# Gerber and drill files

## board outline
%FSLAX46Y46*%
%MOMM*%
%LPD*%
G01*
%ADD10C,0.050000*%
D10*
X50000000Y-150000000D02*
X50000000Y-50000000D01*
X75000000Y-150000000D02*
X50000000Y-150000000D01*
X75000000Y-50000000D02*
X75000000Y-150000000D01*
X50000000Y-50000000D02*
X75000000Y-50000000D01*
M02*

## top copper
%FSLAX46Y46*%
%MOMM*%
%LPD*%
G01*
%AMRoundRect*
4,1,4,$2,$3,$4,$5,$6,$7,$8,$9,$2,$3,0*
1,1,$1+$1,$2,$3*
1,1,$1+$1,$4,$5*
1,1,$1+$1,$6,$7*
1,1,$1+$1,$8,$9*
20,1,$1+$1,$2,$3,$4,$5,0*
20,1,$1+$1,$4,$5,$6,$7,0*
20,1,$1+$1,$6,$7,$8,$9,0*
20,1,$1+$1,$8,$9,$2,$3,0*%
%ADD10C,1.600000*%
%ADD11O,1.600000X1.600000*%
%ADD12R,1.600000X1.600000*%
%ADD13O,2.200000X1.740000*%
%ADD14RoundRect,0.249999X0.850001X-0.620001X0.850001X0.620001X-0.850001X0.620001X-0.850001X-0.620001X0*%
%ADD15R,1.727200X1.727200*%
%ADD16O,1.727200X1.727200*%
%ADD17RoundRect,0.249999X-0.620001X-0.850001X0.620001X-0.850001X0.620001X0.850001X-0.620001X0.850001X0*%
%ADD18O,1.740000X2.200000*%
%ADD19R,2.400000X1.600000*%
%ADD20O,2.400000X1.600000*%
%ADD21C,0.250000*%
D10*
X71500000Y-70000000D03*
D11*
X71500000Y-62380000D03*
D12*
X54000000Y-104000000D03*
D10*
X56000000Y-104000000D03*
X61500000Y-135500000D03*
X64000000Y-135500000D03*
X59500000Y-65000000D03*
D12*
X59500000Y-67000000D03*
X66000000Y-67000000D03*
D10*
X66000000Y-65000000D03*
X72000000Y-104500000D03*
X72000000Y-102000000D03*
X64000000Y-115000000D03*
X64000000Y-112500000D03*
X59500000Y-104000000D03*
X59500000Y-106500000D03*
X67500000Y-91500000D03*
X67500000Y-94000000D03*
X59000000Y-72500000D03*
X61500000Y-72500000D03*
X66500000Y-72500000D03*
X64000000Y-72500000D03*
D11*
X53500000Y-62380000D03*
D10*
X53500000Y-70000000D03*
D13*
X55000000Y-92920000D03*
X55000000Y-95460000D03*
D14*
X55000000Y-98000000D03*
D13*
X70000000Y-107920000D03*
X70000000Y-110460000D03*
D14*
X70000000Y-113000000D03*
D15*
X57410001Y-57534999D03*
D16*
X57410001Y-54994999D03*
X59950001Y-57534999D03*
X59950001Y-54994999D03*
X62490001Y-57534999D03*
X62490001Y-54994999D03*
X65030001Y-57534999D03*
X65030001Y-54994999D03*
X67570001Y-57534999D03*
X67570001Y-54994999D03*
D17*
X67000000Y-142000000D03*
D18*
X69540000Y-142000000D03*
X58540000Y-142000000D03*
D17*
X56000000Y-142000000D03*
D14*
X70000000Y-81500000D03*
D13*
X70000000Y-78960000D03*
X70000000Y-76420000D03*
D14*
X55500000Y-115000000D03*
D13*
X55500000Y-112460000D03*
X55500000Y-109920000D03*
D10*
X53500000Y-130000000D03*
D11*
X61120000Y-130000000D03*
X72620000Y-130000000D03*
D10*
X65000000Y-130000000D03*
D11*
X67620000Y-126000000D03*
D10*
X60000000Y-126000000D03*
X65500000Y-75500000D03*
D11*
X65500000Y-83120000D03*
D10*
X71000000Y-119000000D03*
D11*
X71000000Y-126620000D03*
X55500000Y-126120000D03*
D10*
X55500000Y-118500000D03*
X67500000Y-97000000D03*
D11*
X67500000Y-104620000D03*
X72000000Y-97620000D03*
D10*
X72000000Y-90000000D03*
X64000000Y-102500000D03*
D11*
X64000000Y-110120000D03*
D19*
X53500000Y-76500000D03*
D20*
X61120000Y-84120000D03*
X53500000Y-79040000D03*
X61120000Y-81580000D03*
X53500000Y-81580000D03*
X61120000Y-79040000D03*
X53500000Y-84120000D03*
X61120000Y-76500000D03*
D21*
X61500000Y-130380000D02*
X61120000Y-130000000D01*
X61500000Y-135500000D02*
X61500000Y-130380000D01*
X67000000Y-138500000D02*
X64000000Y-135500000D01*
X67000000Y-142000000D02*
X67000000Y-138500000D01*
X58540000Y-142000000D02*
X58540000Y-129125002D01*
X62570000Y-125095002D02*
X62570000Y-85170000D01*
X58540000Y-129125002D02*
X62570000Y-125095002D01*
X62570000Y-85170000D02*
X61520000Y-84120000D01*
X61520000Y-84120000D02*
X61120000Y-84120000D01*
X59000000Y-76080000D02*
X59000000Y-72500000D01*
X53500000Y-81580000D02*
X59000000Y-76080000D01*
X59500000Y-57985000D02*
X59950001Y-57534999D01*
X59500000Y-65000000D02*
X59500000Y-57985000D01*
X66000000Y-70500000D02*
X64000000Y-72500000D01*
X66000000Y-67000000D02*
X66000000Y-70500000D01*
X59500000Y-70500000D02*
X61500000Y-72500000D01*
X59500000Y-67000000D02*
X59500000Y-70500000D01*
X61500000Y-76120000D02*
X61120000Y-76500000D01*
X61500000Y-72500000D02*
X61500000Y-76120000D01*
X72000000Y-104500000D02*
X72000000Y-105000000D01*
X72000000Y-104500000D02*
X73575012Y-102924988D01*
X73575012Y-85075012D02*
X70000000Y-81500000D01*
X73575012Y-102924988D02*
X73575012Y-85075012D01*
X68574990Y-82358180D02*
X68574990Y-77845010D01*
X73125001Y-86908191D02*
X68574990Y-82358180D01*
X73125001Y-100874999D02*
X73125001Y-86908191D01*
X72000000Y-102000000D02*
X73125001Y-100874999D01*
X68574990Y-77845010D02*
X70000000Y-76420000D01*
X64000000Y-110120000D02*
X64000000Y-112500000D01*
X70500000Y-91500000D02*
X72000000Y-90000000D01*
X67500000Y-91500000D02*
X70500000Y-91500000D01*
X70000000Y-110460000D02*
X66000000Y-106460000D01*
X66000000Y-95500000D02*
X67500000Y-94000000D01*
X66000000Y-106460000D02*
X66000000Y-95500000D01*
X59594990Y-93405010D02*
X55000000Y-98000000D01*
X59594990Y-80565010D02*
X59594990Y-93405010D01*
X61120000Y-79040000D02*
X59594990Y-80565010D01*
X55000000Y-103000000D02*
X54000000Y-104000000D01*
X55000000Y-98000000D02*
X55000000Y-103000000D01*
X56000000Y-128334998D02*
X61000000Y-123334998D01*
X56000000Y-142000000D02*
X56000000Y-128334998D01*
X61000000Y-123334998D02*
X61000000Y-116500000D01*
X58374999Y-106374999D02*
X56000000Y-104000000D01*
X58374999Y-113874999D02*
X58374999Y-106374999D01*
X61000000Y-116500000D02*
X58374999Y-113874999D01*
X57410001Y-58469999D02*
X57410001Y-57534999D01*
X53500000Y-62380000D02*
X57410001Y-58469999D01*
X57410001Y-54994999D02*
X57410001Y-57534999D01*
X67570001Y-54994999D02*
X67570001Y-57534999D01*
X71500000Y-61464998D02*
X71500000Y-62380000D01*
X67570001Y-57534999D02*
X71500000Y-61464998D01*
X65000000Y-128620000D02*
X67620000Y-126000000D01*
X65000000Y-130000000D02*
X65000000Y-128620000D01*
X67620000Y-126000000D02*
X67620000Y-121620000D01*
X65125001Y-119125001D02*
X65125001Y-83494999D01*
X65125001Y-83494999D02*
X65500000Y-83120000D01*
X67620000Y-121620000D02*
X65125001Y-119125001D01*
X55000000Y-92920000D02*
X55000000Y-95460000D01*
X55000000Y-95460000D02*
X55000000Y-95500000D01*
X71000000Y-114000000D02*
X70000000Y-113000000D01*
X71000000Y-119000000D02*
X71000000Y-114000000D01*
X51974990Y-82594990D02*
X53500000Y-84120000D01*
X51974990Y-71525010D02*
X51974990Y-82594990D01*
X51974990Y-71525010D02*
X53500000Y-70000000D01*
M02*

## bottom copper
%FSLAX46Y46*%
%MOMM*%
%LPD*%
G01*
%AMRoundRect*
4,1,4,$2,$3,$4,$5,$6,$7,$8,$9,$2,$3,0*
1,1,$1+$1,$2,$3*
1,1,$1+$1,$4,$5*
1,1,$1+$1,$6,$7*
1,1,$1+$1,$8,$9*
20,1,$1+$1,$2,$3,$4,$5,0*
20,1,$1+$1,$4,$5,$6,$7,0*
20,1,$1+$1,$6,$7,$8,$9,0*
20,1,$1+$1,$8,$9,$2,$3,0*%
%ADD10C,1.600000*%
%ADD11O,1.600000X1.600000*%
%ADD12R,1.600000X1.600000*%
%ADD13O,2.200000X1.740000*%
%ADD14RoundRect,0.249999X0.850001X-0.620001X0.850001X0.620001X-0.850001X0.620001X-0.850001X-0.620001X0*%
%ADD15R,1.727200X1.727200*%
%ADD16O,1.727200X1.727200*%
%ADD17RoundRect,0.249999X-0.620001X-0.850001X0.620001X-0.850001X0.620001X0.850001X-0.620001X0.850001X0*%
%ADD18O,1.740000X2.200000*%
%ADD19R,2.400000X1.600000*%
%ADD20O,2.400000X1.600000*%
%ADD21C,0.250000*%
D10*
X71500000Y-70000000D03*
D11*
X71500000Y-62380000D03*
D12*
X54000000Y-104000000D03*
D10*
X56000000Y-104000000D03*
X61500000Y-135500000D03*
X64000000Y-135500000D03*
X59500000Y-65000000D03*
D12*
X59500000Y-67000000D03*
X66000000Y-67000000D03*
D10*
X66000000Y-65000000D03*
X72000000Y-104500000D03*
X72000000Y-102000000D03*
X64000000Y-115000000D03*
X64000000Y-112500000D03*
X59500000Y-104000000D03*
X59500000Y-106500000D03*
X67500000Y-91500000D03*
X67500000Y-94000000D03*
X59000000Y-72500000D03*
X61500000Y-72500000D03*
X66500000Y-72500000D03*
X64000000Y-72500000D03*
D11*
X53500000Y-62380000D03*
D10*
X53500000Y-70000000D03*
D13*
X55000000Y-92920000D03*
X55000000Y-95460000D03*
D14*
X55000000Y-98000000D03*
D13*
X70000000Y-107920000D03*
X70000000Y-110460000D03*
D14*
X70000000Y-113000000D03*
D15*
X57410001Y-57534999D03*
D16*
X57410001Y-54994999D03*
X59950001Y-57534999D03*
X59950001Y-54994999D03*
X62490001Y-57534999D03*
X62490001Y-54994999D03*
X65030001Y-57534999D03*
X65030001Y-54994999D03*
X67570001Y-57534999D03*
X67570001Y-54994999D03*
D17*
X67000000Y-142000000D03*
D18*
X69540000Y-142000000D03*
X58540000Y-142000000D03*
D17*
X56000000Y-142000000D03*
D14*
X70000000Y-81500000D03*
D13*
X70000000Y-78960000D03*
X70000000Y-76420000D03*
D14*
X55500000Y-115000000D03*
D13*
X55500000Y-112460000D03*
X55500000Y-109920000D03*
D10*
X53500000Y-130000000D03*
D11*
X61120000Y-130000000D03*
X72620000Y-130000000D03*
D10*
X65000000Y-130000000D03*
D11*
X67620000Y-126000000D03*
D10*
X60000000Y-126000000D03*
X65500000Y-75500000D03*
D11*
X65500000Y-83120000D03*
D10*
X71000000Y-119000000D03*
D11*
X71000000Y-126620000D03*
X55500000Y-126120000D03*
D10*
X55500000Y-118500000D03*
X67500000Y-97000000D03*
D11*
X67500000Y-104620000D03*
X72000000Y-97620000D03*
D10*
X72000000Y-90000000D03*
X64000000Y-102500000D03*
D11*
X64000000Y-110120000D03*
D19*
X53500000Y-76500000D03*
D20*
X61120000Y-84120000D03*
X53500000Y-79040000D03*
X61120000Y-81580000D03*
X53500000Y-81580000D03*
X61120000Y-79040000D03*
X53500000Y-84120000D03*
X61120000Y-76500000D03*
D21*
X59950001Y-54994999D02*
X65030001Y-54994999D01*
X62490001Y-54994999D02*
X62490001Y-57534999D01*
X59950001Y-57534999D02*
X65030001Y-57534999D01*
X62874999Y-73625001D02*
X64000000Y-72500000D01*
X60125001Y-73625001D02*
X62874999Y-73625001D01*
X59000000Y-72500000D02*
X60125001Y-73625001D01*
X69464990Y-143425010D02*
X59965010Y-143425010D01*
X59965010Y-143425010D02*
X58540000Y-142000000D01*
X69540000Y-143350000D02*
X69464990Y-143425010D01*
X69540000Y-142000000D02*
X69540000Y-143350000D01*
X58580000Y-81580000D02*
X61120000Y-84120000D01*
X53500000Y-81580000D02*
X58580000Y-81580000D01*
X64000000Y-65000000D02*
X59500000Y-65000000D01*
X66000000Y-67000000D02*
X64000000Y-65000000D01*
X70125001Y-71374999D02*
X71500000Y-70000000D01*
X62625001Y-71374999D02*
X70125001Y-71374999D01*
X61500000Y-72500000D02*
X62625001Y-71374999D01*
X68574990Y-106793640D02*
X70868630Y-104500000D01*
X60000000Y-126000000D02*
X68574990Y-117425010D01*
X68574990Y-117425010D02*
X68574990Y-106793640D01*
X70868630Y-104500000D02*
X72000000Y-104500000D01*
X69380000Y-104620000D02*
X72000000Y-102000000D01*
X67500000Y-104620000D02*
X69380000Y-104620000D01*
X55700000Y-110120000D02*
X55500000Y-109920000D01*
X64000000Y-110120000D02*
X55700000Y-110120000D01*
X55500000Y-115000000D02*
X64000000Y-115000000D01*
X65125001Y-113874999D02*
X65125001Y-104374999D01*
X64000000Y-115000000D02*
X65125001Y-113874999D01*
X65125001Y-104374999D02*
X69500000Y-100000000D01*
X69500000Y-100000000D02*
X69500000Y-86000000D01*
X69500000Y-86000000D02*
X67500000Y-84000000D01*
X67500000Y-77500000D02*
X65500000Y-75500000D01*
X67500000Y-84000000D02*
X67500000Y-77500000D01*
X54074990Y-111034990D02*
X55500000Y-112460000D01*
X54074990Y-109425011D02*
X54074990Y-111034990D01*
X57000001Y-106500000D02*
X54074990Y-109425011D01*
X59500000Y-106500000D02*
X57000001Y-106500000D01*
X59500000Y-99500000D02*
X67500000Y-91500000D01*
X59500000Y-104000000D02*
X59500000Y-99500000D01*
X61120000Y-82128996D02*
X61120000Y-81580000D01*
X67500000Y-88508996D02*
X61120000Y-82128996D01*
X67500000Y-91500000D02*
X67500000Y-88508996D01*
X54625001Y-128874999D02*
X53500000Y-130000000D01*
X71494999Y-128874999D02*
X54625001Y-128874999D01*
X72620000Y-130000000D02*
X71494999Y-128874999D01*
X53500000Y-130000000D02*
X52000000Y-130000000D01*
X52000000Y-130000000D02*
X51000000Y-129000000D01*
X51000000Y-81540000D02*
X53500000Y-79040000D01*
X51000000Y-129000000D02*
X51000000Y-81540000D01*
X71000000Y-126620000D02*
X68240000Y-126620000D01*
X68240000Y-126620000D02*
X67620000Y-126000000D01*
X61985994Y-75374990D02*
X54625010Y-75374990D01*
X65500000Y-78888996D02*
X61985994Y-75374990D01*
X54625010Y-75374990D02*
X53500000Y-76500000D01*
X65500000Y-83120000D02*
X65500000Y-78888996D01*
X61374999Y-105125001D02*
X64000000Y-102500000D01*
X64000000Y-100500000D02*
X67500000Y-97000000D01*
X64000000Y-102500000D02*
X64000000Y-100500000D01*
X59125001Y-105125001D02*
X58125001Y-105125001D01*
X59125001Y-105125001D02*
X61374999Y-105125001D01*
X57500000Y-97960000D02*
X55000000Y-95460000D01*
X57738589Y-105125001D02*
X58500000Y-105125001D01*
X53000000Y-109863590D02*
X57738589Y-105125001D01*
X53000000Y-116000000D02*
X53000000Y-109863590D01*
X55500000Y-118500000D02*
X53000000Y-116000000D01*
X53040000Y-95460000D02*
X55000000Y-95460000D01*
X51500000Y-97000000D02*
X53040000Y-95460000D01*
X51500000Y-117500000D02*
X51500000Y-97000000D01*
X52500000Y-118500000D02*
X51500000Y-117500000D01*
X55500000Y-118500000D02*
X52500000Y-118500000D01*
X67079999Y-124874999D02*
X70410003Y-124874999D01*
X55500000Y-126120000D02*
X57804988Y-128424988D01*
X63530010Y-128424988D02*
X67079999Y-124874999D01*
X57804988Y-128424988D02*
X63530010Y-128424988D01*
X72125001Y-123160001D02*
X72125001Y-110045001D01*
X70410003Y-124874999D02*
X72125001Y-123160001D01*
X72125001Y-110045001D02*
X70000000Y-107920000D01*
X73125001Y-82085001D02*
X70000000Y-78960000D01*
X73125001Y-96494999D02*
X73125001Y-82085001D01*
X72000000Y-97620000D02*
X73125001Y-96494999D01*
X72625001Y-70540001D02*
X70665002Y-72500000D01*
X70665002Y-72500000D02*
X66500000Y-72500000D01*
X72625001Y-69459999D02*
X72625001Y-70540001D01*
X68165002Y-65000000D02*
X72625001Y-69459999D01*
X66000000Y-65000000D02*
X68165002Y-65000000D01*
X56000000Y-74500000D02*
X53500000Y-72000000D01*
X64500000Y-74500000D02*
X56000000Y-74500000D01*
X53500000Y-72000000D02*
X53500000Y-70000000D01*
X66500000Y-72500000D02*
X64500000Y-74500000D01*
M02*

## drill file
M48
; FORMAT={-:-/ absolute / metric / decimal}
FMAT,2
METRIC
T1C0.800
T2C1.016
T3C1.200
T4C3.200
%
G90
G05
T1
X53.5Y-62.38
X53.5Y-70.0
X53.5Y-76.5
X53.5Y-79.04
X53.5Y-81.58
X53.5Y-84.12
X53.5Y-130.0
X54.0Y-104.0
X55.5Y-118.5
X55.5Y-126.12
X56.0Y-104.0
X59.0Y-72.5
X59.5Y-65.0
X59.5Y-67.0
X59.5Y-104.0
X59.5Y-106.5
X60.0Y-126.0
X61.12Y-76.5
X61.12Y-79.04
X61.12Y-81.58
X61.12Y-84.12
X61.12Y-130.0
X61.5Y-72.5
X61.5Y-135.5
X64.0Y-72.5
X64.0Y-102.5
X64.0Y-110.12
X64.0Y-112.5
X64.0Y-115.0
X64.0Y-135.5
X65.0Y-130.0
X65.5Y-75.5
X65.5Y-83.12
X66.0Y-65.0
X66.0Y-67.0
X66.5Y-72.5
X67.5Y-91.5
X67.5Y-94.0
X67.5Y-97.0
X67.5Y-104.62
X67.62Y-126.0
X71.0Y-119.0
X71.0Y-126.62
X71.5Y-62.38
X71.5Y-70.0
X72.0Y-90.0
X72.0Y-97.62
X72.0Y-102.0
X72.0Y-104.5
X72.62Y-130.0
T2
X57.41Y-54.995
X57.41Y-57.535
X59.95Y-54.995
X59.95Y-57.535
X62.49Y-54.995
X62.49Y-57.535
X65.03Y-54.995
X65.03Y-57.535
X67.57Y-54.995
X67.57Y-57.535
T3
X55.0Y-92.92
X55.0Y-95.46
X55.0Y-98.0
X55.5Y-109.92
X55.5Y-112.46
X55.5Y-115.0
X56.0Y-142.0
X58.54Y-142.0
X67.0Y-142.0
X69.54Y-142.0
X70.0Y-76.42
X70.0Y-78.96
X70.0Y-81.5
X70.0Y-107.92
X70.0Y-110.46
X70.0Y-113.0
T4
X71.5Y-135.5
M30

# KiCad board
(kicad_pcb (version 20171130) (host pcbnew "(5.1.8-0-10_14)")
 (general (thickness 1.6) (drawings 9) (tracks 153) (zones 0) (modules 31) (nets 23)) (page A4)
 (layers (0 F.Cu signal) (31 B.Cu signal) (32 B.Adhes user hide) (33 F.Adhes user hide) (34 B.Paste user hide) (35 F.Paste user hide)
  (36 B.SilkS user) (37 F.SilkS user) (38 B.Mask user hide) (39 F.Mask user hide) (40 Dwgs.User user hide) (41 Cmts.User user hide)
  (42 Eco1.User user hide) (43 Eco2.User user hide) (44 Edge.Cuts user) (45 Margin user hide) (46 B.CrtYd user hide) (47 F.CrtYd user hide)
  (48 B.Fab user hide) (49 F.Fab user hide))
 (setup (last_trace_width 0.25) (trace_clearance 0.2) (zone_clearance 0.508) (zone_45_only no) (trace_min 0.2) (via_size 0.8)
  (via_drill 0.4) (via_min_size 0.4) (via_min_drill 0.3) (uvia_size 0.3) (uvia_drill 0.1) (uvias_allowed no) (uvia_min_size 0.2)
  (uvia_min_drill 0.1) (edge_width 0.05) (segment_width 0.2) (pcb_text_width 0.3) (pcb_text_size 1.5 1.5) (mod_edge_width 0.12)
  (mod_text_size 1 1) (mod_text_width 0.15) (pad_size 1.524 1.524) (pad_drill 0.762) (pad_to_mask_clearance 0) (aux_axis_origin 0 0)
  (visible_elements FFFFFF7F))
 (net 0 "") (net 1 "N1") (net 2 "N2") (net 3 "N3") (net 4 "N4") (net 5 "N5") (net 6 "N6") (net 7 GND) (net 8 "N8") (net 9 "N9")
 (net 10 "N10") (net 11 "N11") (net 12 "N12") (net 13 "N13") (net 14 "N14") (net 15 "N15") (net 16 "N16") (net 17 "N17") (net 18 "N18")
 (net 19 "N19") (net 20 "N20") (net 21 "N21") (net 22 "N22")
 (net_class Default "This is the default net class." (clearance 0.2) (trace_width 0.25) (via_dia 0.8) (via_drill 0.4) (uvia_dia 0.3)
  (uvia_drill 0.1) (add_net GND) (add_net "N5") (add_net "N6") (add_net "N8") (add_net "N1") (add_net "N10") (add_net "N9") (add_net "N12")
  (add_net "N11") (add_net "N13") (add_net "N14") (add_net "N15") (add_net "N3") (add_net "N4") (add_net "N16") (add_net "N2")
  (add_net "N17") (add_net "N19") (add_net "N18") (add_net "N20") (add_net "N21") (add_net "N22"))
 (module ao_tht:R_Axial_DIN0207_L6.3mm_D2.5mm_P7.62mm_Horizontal (layer F.Cu) (at 71.5 70 90)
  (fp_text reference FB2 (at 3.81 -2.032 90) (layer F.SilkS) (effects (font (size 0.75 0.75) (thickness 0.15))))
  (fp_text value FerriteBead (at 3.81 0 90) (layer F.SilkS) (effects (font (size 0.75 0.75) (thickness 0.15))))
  (pad 1 thru_hole circle (at 0 0 90) (size 1.6 1.6) (drill 0.8) (layers *.Cu *.Mask) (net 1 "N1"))
  (pad 2 thru_hole oval (at 7.62 0 90) (size 1.6 1.6) (drill 0.8) (layers *.Cu *.Mask) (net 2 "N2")))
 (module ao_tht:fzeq (layer B.Cu) (at 62 63 180)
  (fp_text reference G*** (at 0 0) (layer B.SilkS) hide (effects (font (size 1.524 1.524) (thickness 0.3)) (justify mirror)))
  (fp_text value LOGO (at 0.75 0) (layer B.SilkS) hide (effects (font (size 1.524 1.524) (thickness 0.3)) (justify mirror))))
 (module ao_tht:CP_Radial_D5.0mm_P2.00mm (layer F.Cu) (at 54 104)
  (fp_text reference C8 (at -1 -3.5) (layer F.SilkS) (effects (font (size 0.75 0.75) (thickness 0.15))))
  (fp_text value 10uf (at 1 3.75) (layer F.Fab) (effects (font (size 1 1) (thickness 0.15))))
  (pad 1 thru_hole rect (at 0 0) (size 1.6 1.6) (drill 0.8) (layers *.Cu *.Mask) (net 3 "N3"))
  (pad 2 thru_hole circle (at 2 0) (size 1.6 1.6) (drill 0.8) (layers *.Cu *.Mask) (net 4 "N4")))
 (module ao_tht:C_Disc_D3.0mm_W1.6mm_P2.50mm (layer F.Cu) (at 61.5 135.5)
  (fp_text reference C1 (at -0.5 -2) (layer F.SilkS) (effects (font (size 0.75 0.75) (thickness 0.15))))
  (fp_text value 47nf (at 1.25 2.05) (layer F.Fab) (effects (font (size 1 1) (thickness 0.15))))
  (pad 1 thru_hole circle (at 0 0) (size 1.6 1.6) (drill 0.8) (layers *.Cu *.Mask) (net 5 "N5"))
  (pad 2 thru_hole circle (at 2.5 0) (size 1.6 1.6) (drill 0.8) (layers *.Cu *.Mask) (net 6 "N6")))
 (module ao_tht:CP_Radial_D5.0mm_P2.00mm (layer F.Cu) (at 59.5 67 90)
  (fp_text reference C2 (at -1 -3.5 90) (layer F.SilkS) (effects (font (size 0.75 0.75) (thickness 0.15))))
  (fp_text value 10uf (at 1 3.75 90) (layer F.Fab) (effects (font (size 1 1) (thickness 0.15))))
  (pad 2 thru_hole circle (at 2 0 90) (size 1.6 1.6) (drill 0.8) (layers *.Cu *.Mask) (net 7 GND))
  (pad 1 thru_hole rect (at 0 0 90) (size 1.6 1.6) (drill 0.8) (layers *.Cu *.Mask) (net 1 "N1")))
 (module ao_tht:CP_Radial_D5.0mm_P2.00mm (layer F.Cu) (at 66 67 90)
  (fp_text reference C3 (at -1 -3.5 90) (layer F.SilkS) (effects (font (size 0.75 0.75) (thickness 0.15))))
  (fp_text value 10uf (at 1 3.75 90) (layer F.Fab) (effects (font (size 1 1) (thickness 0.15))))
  (pad 1 thru_hole rect (at 0 0 90) (size 1.6 1.6) (drill 0.8) (layers *.Cu *.Mask) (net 7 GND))
  (pad 2 thru_hole circle (at 2 0 90) (size 1.6 1.6) (drill 0.8) (layers *.Cu *.Mask) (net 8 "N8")))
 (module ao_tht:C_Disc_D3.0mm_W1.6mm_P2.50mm (layer F.Cu) (at 72 102 270)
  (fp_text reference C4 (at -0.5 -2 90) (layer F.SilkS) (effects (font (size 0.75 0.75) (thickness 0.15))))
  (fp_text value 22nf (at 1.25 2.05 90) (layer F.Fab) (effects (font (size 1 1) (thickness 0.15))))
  (pad 2 thru_hole circle (at 2.5 0 270) (size 1.6 1.6) (drill 0.8) (layers *.Cu *.Mask) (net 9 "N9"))
  (pad 1 thru_hole circle (at 0 0 270) (size 1.6 1.6) (drill 0.8) (layers *.Cu *.Mask) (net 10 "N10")))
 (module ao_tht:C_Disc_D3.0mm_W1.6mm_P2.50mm (layer F.Cu) (at 64 112.5 270)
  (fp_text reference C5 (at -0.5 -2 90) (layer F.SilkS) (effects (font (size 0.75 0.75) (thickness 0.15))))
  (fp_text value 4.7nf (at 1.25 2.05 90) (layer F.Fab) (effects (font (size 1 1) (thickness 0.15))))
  (pad 2 thru_hole circle (at 2.5 0 270) (size 1.6 1.6) (drill 0.8) (layers *.Cu *.Mask) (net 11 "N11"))
  (pad 1 thru_hole circle (at 0 0 270) (size 1.6 1.6) (drill 0.8) (layers *.Cu *.Mask) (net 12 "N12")))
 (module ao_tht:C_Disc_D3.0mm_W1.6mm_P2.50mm (layer F.Cu) (at 59.5 104 270)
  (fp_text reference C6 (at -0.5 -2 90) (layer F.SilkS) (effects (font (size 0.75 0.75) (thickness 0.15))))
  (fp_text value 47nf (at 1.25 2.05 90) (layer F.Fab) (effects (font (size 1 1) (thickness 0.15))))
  (pad 1 thru_hole circle (at 0 0 270) (size 1.6 1.6) (drill 0.8) (layers *.Cu *.Mask) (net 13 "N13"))
  (pad 2 thru_hole circle (at 2.5 0 270) (size 1.6 1.6) (drill 0.8) (layers *.Cu *.Mask) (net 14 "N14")))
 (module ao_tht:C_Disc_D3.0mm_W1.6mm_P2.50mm (layer F.Cu) (at 67.5 91.5 270)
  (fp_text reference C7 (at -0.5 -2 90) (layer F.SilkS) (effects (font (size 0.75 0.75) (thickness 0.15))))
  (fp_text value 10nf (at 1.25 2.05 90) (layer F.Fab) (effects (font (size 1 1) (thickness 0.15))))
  (pad 1 thru_hole circle (at 0 0 270) (size 1.6 1.6) (drill 0.8) (layers *.Cu *.Mask) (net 13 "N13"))
  (pad 2 thru_hole circle (at 2.5 0 270) (size 1.6 1.6) (drill 0.8) (layers *.Cu *.Mask) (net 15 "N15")))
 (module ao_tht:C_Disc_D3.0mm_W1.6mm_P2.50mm (layer F.Cu) (at 59 72.5)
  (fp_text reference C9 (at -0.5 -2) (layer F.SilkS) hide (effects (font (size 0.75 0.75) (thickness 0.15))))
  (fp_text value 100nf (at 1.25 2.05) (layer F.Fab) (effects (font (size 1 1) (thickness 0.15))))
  (pad 1 thru_hole circle (at 0 0) (size 1.6 1.6) (drill 0.8) (layers *.Cu *.Mask) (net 7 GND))
  (pad 2 thru_hole circle (at 2.5 0) (size 1.6 1.6) (drill 0.8) (layers *.Cu *.Mask) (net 1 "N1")))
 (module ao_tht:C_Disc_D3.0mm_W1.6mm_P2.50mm (layer F.Cu) (at 64 72.5)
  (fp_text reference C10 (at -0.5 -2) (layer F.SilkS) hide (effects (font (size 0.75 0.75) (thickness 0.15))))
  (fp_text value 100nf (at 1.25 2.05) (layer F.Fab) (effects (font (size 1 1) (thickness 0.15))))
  (pad 2 thru_hole circle (at 2.5 0) (size 1.6 1.6) (drill 0.8) (layers *.Cu *.Mask) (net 8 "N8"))
  (pad 1 thru_hole circle (at 0 0) (size 1.6 1.6) (drill 0.8) (layers *.Cu *.Mask) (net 7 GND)))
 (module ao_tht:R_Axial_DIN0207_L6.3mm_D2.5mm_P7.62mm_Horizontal (layer F.Cu) (at 53.5 70 90)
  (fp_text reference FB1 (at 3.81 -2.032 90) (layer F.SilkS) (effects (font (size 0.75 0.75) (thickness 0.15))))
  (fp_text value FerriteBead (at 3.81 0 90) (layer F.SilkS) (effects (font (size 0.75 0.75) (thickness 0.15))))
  (pad 2 thru_hole oval (at 7.62 0 90) (size 1.6 1.6) (drill 0.8) (layers *.Cu *.Mask) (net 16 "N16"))
  (pad 1 thru_hole circle (at 0 0 90) (size 1.6 1.6) (drill 0.8) (layers *.Cu *.Mask) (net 8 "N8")))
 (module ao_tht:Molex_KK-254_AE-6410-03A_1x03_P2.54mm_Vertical (layer B.Cu) (at 55 98 90)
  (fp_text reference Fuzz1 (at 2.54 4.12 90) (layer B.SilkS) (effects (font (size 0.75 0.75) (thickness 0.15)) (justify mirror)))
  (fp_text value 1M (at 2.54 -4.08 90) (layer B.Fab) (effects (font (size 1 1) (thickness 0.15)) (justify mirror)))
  (pad 3 thru_hole oval (at 5.08 0 90) (size 1.74 2.2) (drill 1.2) (layers *.Cu *.Mask) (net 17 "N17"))
  (pad 2 thru_hole oval (at 2.54 0 90) (size 1.74 2.2) (drill 1.2) (layers *.Cu *.Mask) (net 17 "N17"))
  (pad 1 thru_hole roundrect (at 0 0 90) (size 1.74 2.2) (drill 1.2) (layers *.Cu *.Mask) (roundrect_rratio 0.1436775862068966) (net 3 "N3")))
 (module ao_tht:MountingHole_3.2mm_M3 (layer F.Cu) (at 71.5 135.5)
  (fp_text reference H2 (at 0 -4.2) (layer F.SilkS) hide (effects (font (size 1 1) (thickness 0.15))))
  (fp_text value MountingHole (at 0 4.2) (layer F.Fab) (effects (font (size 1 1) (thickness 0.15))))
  (pad 1 np_thru_hole circle (at 0 0) (size 3.2 3.2) (drill 3.2) (layers *.Cu *.Mask)))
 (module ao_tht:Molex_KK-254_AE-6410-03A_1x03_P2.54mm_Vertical (layer B.Cu) (at 70 113 90)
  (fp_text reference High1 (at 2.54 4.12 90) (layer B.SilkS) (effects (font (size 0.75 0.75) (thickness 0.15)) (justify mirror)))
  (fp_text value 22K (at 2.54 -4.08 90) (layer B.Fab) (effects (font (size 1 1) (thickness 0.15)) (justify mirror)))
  (pad 3 thru_hole oval (at 5.08 0 90) (size 1.74 2.2) (drill 1.2) (layers *.Cu *.Mask) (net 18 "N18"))
  (pad 2 thru_hole oval (at 2.54 0 90) (size 1.74 2.2) (drill 1.2) (layers *.Cu *.Mask) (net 15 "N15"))
  (pad 1 thru_hole roundrect (at 0 0 90) (size 1.74 2.2) (drill 1.2) (layers *.Cu *.Mask) (roundrect_rratio 0.1436775862068966)
   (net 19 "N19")))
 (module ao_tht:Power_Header (layer F.Cu) (at 57.410001 57.534999 90)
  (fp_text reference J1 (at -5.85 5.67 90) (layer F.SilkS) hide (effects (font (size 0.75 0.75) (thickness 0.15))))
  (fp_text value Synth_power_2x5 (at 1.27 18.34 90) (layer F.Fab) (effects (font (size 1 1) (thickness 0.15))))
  (pad 1 thru_hole rect (at 0 0 90) (size 1.7272 1.7272) (drill 1.016) (layers *.Cu *.Mask) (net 16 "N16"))
  (pad 2 thru_hole oval (at 2.54 0 90) (size 1.7272 1.7272) (drill 1.016) (layers *.Cu *.Mask) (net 16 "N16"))
  (pad 3 thru_hole oval (at 0 2.54 90) (size 1.7272 1.7272) (drill 1.016) (layers *.Cu *.Mask) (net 7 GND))
  (pad 4 thru_hole oval (at 2.54 2.54 90) (size 1.7272 1.7272) (drill 1.016) (layers *.Cu *.Mask) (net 7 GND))
  (pad 5 thru_hole oval (at 0 5.08 90) (size 1.7272 1.7272) (drill 1.016) (layers *.Cu *.Mask) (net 7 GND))
  (pad 6 thru_hole oval (at 2.54 5.08 90) (size 1.7272 1.7272) (drill 1.016) (layers *.Cu *.Mask) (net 7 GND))
  (pad 7 thru_hole oval (at 0 7.62 90) (size 1.7272 1.7272) (drill 1.016) (layers *.Cu *.Mask) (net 7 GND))
  (pad 8 thru_hole oval (at 2.54 7.62 90) (size 1.7272 1.7272) (drill 1.016) (layers *.Cu *.Mask) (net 7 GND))
  (pad 9 thru_hole oval (at 0 10.16 90) (size 1.7272 1.7272) (drill 1.016) (layers *.Cu *.Mask) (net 2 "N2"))
  (pad 10 thru_hole oval (at 2.54 10.16 90) (size 1.7272 1.7272) (drill 1.016) (layers *.Cu *.Mask) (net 2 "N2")))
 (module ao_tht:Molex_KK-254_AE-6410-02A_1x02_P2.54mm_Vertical (layer B.Cu) (at 67 142)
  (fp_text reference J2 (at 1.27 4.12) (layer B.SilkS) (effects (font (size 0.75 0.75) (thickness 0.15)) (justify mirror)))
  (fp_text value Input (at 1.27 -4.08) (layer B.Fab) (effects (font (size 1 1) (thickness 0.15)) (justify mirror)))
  (pad 1 thru_hole roundrect (at 0 0) (size 1.74 2.2) (drill 1.2) (layers *.Cu *.Mask) (roundrect_rratio 0.1436775862068966) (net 6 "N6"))
  (pad 2 thru_hole oval (at 2.54 0) (size 1.74 2.2) (drill 1.2) (layers *.Cu *.Mask) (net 7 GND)))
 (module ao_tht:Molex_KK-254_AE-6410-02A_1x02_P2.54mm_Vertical (layer B.Cu) (at 56 142)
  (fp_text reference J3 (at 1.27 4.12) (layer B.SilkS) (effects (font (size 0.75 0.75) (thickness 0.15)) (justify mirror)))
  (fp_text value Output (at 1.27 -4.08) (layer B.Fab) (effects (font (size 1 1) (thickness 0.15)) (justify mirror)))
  (pad 2 thru_hole oval (at 2.54 0) (size 1.74 2.2) (drill 1.2) (layers *.Cu *.Mask) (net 7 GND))
  (pad 1 thru_hole roundrect (at 0 0) (size 1.74 2.2) (drill 1.2) (layers *.Cu *.Mask) (roundrect_rratio 0.1436775862068966) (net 4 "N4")))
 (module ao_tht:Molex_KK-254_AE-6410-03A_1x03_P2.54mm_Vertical (layer B.Cu) (at 70 81.5 90)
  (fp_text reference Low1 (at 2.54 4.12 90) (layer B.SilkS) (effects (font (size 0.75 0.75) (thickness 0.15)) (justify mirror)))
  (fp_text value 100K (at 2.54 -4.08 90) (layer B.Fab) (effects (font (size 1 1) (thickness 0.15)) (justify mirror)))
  (pad 1 thru_hole roundrect (at 0 0 90) (size 1.74 2.2) (drill 1.2) (layers *.Cu *.Mask) (roundrect_rratio 0.1436775862068966) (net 9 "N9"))
  (pad 2 thru_hole oval (at 2.54 0 90) (size 1.74 2.2) (drill 1.2) (layers *.Cu *.Mask) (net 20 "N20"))
  (pad 3 thru_hole oval (at 5.08 0 90) (size 1.74 2.2) (drill 1.2) (layers *.Cu *.Mask) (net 10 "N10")))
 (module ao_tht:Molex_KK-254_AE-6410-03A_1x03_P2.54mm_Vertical (layer B.Cu) (at 55.5 115 90)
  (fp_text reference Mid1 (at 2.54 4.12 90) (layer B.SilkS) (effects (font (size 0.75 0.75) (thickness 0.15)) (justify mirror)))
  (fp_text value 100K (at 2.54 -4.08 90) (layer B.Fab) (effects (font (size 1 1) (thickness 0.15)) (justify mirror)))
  (pad 1 thru_hole roundrect (at 0 0 90) (size 1.74 2.2) (drill 1.2) (layers *.Cu *.Mask) (roundrect_rratio 0.1436775862068966)
   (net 11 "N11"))
  (pad 2 thru_hole oval (at 2.54 0 90) (size 1.74 2.2) (drill 1.2) (layers *.Cu *.Mask) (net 14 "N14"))
  (pad 3 thru_hole oval (at 5.08 0 90) (size 1.74 2.2) (drill 1.2) (layers *.Cu *.Mask) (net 12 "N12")))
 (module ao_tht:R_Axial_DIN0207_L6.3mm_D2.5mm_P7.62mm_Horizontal (layer F.Cu) (at 53.5 130)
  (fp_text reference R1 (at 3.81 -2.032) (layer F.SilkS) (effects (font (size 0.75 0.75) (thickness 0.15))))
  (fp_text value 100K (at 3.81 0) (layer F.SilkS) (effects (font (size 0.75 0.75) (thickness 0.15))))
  (pad 1 thru_hole circle (at 0 0) (size 1.6 1.6) (drill 0.8) (layers *.Cu *.Mask) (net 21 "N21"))
  (pad 2 thru_hole oval (at 7.62 0) (size 1.6 1.6) (drill 0.8) (layers *.Cu *.Mask) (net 5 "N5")))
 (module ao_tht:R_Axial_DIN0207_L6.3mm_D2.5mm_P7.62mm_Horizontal (layer F.Cu) (at 65 130)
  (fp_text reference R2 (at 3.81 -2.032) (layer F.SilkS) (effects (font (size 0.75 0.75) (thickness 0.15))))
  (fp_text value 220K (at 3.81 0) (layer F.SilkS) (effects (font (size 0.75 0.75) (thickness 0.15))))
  (pad 2 thru_hole oval (at 7.62 0) (size 1.6 1.6) (drill 0.8) (layers *.Cu *.Mask) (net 21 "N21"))
  (pad 1 thru_hole circle (at 0 0) (size 1.6 1.6) (drill 0.8) (layers *.Cu *.Mask) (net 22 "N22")))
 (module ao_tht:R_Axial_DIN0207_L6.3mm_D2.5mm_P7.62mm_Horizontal (layer F.Cu) (at 60 126)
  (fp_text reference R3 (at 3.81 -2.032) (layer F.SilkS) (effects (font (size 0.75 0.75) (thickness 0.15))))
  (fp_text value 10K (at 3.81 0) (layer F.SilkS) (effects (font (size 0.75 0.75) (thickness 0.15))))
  (pad 2 thru_hole oval (at 7.62 0) (size 1.6 1.6) (drill 0.8) (layers *.Cu *.Mask) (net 22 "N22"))
  (pad 1 thru_hole circle (at 0 0) (size 1.6 1.6) (drill 0.8) (layers *.Cu *.Mask) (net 9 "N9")))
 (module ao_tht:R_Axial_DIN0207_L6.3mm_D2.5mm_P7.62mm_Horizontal (layer F.Cu) (at 65.5 75.5 270)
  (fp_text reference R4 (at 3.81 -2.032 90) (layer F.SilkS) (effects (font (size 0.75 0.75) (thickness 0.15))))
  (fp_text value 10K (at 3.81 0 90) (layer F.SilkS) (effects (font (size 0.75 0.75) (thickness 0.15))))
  (pad 1 thru_hole circle (at 0 0 270) (size 1.6 1.6) (drill 0.8) (layers *.Cu *.Mask) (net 11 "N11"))
  (pad 2 thru_hole oval (at 7.62 0 270) (size 1.6 1.6) (drill 0.8) (layers *.Cu *.Mask) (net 22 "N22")))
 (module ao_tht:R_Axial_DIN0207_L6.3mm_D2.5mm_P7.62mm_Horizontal (layer F.Cu) (at 71 119 270)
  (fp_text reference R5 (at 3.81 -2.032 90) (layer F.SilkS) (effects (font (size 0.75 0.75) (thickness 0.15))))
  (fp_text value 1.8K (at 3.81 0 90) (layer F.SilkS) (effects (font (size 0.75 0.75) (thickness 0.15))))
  (pad 1 thru_hole circle (at 0 0 270) (size 1.6 1.6) (drill 0.8) (layers *.Cu *.Mask) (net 19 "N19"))
  (pad 2 thru_hole oval (at 7.62 0 270) (size 1.6 1.6) (drill 0.8) (layers *.Cu *.Mask) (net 22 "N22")))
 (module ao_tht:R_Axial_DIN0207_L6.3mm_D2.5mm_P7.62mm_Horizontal (layer F.Cu) (at 55.5 118.5 270)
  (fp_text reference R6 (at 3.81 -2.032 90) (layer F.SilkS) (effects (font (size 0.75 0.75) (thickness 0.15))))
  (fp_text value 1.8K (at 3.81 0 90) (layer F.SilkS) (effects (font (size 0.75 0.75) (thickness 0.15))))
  (pad 2 thru_hole oval (at 7.62 0 270) (size 1.6 1.6) (drill 0.8) (layers *.Cu *.Mask) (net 18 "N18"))
  (pad 1 thru_hole circle (at 0 0 270) (size 1.6 1.6) (drill 0.8) (layers *.Cu *.Mask) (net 17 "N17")))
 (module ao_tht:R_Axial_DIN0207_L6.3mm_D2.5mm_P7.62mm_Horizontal (layer F.Cu) (at 67.5 97 270)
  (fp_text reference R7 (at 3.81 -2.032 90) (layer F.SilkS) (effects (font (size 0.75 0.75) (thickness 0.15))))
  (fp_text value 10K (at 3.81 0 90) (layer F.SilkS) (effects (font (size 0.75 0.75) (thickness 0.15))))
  (pad 1 thru_hole circle (at 0 0 270) (size 1.6 1.6) (drill 0.8) (layers *.Cu *.Mask) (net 17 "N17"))
  (pad 2 thru_hole oval (at 7.62 0 270) (size 1.6 1.6) (drill 0.8) (layers *.Cu *.Mask) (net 10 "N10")))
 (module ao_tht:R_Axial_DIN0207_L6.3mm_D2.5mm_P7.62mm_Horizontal (layer F.Cu) (at 72 90 270)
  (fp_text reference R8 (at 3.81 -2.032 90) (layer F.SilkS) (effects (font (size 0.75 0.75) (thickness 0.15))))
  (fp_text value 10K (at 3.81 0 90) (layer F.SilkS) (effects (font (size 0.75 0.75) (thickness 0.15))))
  (pad 2 thru_hole oval (at 7.62 0 270) (size 1.6 1.6) (drill 0.8) (layers *.Cu *.Mask) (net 20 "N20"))
  (pad 1 thru_hole circle (at 0 0 270) (size 1.6 1.6) (drill 0.8) (layers *.Cu *.Mask) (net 13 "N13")))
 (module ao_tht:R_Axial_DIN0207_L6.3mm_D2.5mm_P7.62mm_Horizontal (layer F.Cu) (at 64 102.5 270)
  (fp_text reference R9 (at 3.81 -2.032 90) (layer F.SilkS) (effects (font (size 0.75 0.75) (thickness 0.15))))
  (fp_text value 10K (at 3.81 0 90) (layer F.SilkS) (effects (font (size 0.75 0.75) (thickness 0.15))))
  (pad 1 thru_hole circle (at 0 0 270) (size 1.6 1.6) (drill 0.8) (layers *.Cu *.Mask) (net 17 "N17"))
  (pad 2 thru_hole oval (at 7.62 0 270) (size 1.6 1.6) (drill 0.8) (layers *.Cu *.Mask) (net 12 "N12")))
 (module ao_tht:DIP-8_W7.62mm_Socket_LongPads (layer F.Cu) (at 53.5 76.5)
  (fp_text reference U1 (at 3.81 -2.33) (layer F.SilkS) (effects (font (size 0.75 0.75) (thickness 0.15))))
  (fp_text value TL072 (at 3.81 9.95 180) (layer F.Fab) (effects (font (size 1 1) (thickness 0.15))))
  (pad 1 thru_hole rect (at 0 0) (size 2.4 1.6) (drill 0.8) (layers *.Cu *.Mask) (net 22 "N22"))
  (pad 5 thru_hole oval (at 7.62 7.62) (size 2.4 1.6) (drill 0.8) (layers *.Cu *.Mask) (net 7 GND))
  (pad 2 thru_hole oval (at 0 2.54) (size 2.4 1.6) (drill 0.8) (layers *.Cu *.Mask) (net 21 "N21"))
  (pad 6 thru_hole oval (at 7.62 5.08) (size 2.4 1.6) (drill 0.8) (layers *.Cu *.Mask) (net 13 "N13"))
  (pad 3 thru_hole oval (at 0 5.08) (size 2.4 1.6) (drill 0.8) (layers *.Cu *.Mask) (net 7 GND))
  (pad 7 thru_hole oval (at 7.62 2.54) (size 2.4 1.6) (drill 0.8) (layers *.Cu *.Mask) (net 3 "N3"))
  (pad 4 thru_hole oval (at 0 7.62) (size 2.4 1.6) (drill 0.8) (layers *.Cu *.Mask) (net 8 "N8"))
  (pad 8 thru_hole oval (at 7.62 0) (size 2.4 1.6) (drill 0.8) (layers *.Cu *.Mask) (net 1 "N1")))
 (gr_line (start 50 150) (end 50 50) (layer Edge.Cuts) (width 0.05))
 (gr_line (start 75 150) (end 50 150) (layer Edge.Cuts) (width 0.05))
 (gr_line (start 75 50) (end 75 150) (layer Edge.Cuts) (width 0.05))
 (gr_line (start 50 50) (end 75 50) (layer Edge.Cuts) (width 0.05))
 (segment (start 61.5 130.38) (end 61.12 130) (width 0.25) (layer F.Cu) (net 5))
 (segment (start 61.5 135.5) (end 61.5 130.38) (width 0.25) (layer F.Cu) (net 5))
 (segment (start 67 138.5) (end 64 135.5) (width 0.25) (layer F.Cu) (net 6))
 (segment (start 67 142) (end 67 138.5) (width 0.25) (layer F.Cu) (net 6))
 (segment (start 58.54 142) (end 58.54 129.125002) (width 0.25) (layer F.Cu) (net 7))
 (segment (start 62.57 125.095002) (end 62.57 85.17) (width 0.25) (layer F.Cu) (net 7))
 (segment (start 58.54 129.125002) (end 62.57 125.095002) (width 0.25) (layer F.Cu) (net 7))
 (segment (start 62.57 85.17) (end 61.52 84.12) (width 0.25) (layer F.Cu) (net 7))
 (segment (start 61.52 84.12) (end 61.12 84.12) (width 0.25) (layer F.Cu) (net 7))
 (segment (start 59 76.08) (end 59 72.5) (width 0.25) (layer F.Cu) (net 7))
 (segment (start 53.5 81.58) (end 59 76.08) (width 0.25) (layer F.Cu) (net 7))
 (segment (start 59.950001 54.994999) (end 65.030001 54.994999) (width 0.25) (layer B.Cu) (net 7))
 (segment (start 62.490001 54.994999) (end 62.490001 57.534999) (width 0.25) (layer B.Cu) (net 7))
 (segment (start 59.950001 57.534999) (end 65.030001 57.534999) (width 0.25) (layer B.Cu) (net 7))
 (segment (start 62.874999 73.625001) (end 64 72.5) (width 0.25) (layer B.Cu) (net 7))
 (segment (start 60.125001 73.625001) (end 62.874999 73.625001) (width 0.25) (layer B.Cu) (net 7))
 (segment (start 59 72.5) (end 60.125001 73.625001) (width 0.25) (layer B.Cu) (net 7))
 (segment (start 69.46499 143.42501) (end 59.96501 143.42501) (width 0.25) (layer B.Cu) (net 7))
 (segment (start 59.96501 143.42501) (end 58.54 142) (width 0.25) (layer B.Cu) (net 7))
 (segment (start 69.54 143.35) (end 69.46499 143.42501) (width 0.25) (layer B.Cu) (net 7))
 (segment (start 69.54 142) (end 69.54 143.35) (width 0.25) (layer B.Cu) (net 7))
 (segment (start 58.58 81.58) (end 61.12 84.12) (width 0.25) (layer B.Cu) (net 7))
 (segment (start 53.5 81.58) (end 58.58 81.58) (width 0.25) (layer B.Cu) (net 7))
 (segment (start 59.5 57.985) (end 59.950001 57.534999) (width 0.25) (layer F.Cu) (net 7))
 (segment (start 59.5 65) (end 59.5 57.985) (width 0.25) (layer F.Cu) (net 7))
 (segment (start 64 65) (end 59.5 65) (width 0.25) (layer B.Cu) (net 7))
 (segment (start 66 67) (end 64 65) (width 0.25) (layer B.Cu) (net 7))
 (segment (start 66 70.5) (end 64 72.5) (width 0.25) (layer F.Cu) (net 7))
 (segment (start 66 67) (end 66 70.5) (width 0.25) (layer F.Cu) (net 7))
 (segment (start 59.5 70.5) (end 61.5 72.5) (width 0.25) (layer F.Cu) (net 1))
 (segment (start 59.5 67) (end 59.5 70.5) (width 0.25) (layer F.Cu) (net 1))
 (segment (start 61.5 76.12) (end 61.12 76.5) (width 0.25) (layer F.Cu) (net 1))
 (segment (start 61.5 72.5) (end 61.5 76.12) (width 0.25) (layer F.Cu) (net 1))
 (segment (start 70.125001 71.374999) (end 71.5 70) (width 0.25) (layer B.Cu) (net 1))
 (segment (start 62.625001 71.374999) (end 70.125001 71.374999) (width 0.25) (layer B.Cu) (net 1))
 (segment (start 61.5 72.5) (end 62.625001 71.374999) (width 0.25) (layer B.Cu) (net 1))
 (segment (start 72 104.5) (end 72 105) (width 0.25) (layer F.Cu) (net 9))
 (segment (start 72 104.5) (end 73.575012 102.924988) (width 0.25) (layer F.Cu) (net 9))
 (segment (start 73.575012 85.075012) (end 70 81.5) (width 0.25) (layer F.Cu) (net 9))
 (segment (start 73.575012 102.924988) (end 73.575012 85.075012) (width 0.25) (layer F.Cu) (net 9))
 (segment (start 68.57499 106.79364) (end 70.86863 104.5) (width 0.25) (layer B.Cu) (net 9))
 (segment (start 60 126) (end 68.57499 117.42501) (width 0.25) (layer B.Cu) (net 9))
 (segment (start 68.57499 117.42501) (end 68.57499 106.79364) (width 0.25) (layer B.Cu) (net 9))
 (segment (start 70.86863 104.5) (end 72 104.5) (width 0.25) (layer B.Cu) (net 9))
 (segment (start 68.57499 82.35818) (end 68.57499 77.84501) (width 0.25) (layer F.Cu) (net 10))
 (segment (start 73.125001 86.908191) (end 68.57499 82.35818) (width 0.25) (layer F.Cu) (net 10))
 (segment (start 73.125001 100.874999) (end 73.125001 86.908191) (width 0.25) (layer F.Cu) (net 10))
 (segment (start 72 102) (end 73.125001 100.874999) (width 0.25) (layer F.Cu) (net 10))
 (segment (start 68.57499 77.84501) (end 70 76.42) (width 0.25) (layer F.Cu) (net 10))
 (segment (start 69.38 104.62) (end 72 102) (width 0.25) (layer B.Cu) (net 10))
 (segment (start 67.5 104.62) (end 69.38 104.62) (width 0.25) (layer B.Cu) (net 10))
 (segment (start 55.7 110.12) (end 55.5 109.92) (width 0.25) (layer B.Cu) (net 12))
 (segment (start 64 110.12) (end 55.7 110.12) (width 0.25) (layer B.Cu) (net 12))
 (segment (start 64 110.12) (end 64 112.5) (width 0.25) (layer F.Cu) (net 12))
 (segment (start 55.5 115) (end 64 115) (width 0.25) (layer B.Cu) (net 11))
 (segment (start 65.125001 113.874999) (end 65.125001 104.374999) (width 0.25) (layer B.Cu) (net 11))
 (segment (start 64 115) (end 65.125001 113.874999) (width 0.25) (layer B.Cu) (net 11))
 (segment (start 65.125001 104.374999) (end 69.5 100) (width 0.25) (layer B.Cu) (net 11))
 (segment (start 69.5 100) (end 69.5 86) (width 0.25) (layer B.Cu) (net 11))
 (segment (start 69.5 86) (end 67.5 84) (width 0.25) (layer B.Cu) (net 11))
 (segment (start 67.5 77.5) (end 65.5 75.5) (width 0.25) (layer B.Cu) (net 11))
 (segment (start 67.5 84) (end 67.5 77.5) (width 0.25) (layer B.Cu) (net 11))
 (segment (start 54.07499 111.03499) (end 55.5 112.46) (width 0.25) (layer B.Cu) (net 14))
 (segment (start 54.07499 109.425011) (end 54.07499 111.03499) (width 0.25) (layer B.Cu) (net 14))
 (segment (start 57.000001 106.5) (end 54.07499 109.425011) (width 0.25) (layer B.Cu) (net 14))
 (segment (start 59.5 106.5) (end 57.000001 106.5) (width 0.25) (layer B.Cu) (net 14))
 (segment (start 59.5 99.5) (end 67.5 91.5) (width 0.25) (layer B.Cu) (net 13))
 (segment (start 59.5 104) (end 59.5 99.5) (width 0.25) (layer B.Cu) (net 13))
 (segment (start 61.12 82.128996) (end 61.12 81.58) (width 0.25) (layer B.Cu) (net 13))
 (segment (start 67.5 88.508996) (end 61.12 82.128996) (width 0.25) (layer B.Cu) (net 13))
 (segment (start 67.5 91.5) (end 67.5 88.508996) (width 0.25) (layer B.Cu) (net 13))
 (segment (start 70.5 91.5) (end 72 90) (width 0.25) (layer F.Cu) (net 13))
 (segment (start 67.5 91.5) (end 70.5 91.5) (width 0.25) (layer F.Cu) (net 13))
 (segment (start 70 110.46) (end 66 106.46) (width 0.25) (layer F.Cu) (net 15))
 (segment (start 66 95.5) (end 67.5 94) (width 0.25) (layer F.Cu) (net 15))
 (segment (start 66 106.46) (end 66 95.5) (width 0.25) (layer F.Cu) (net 15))
 (segment (start 59.59499 93.40501) (end 55 98) (width 0.25) (layer F.Cu) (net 3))
 (segment (start 59.59499 80.56501) (end 59.59499 93.40501) (width 0.25) (layer F.Cu) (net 3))
 (segment (start 61.12 79.04) (end 59.59499 80.56501) (width 0.25) (layer F.Cu) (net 3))
 (segment (start 55 103) (end 54 104) (width 0.25) (layer F.Cu) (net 3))
 (segment (start 55 98) (end 55 103) (width 0.25) (layer F.Cu) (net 3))
 (segment (start 56 128.334998) (end 61 123.334998) (width 0.25) (layer F.Cu) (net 4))
 (segment (start 56 142) (end 56 128.334998) (width 0.25) (layer F.Cu) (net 4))
 (segment (start 61 123.334998) (end 61 116.5) (width 0.25) (layer F.Cu) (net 4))
 (segment (start 58.374999 106.374999) (end 56 104) (width 0.25) (layer F.Cu) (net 4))
 (segment (start 58.374999 113.874999) (end 58.374999 106.374999) (width 0.25) (layer F.Cu) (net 4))
 (segment (start 61 116.5) (end 58.374999 113.874999) (width 0.25) (layer F.Cu) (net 4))
 (segment (start 57.410001 58.469999) (end 57.410001 57.534999) (width 0.25) (layer F.Cu) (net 16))
 (segment (start 53.5 62.38) (end 57.410001 58.469999) (width 0.25) (layer F.Cu) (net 16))
 (segment (start 57.410001 54.994999) (end 57.410001 57.534999) (width 0.25) (layer F.Cu) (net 16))
 (segment (start 67.570001 54.994999) (end 67.570001 57.534999) (width 0.25) (layer F.Cu) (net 2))
 (segment (start 71.5 61.464998) (end 71.5 62.38) (width 0.25) (layer F.Cu) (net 2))
 (segment (start 67.570001 57.534999) (end 71.5 61.464998) (width 0.25) (layer F.Cu) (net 2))
 (segment (start 54.625001 128.874999) (end 53.5 130) (width 0.25) (layer B.Cu) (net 21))
 (segment (start 71.494999 128.874999) (end 54.625001 128.874999) (width 0.25) (layer B.Cu) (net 21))
 (segment (start 72.62 130) (end 71.494999 128.874999) (width 0.25) (layer B.Cu) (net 21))
 (segment (start 53.5 130) (end 52 130) (width 0.25) (layer B.Cu) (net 21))
 (segment (start 52 130) (end 51 129) (width 0.25) (layer B.Cu) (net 21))
 (segment (start 51 81.54) (end 53.5 79.04) (width 0.25) (layer B.Cu) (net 21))
 (segment (start 51 129) (end 51 81.54) (width 0.25) (layer B.Cu) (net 21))
 (segment (start 65 128.62) (end 67.62 126) (width 0.25) (layer F.Cu) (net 22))
 (segment (start 65 130) (end 65 128.62) (width 0.25) (layer F.Cu) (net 22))
 (segment (start 67.62 126) (end 67.62 121.62) (width 0.25) (layer F.Cu) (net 22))
 (segment (start 65.125001 119.125001) (end 65.125001 83.494999) (width 0.25) (layer F.Cu) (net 22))
 (segment (start 65.125001 83.494999) (end 65.5 83.12) (width 0.25) (layer F.Cu) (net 22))
 (segment (start 67.62 121.62) (end 65.125001 119.125001) (width 0.25) (layer F.Cu) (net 22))
 (segment (start 71 126.62) (end 68.24 126.62) (width 0.25) (layer B.Cu) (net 22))
 (segment (start 68.24 126.62) (end 67.62 126) (width 0.25) (layer B.Cu) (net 22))
 (segment (start 61.985994 75.37499) (end 54.62501 75.37499) (width 0.25) (layer B.Cu) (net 22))
 (segment (start 65.5 78.888996) (end 61.985994 75.37499) (width 0.25) (layer B.Cu) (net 22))
 (segment (start 54.62501 75.37499) (end 53.5 76.5) (width 0.25) (layer B.Cu) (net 22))
 (segment (start 65.5 83.12) (end 65.5 78.888996) (width 0.25) (layer B.Cu) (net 22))
 (segment (start 55 92.92) (end 55 95.46) (width 0.25) (layer F.Cu) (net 17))
 (segment (start 61.374999 105.125001) (end 64 102.5) (width 0.25) (layer B.Cu) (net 17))
 (segment (start 64 100.5) (end 67.5 97) (width 0.25) (layer B.Cu) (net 17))
 (segment (start 64 102.5) (end 64 100.5) (width 0.25) (layer B.Cu) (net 17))
 (segment (start 55 95.46) (end 55 95.5) (width 0.25) (layer F.Cu) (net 17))
 (segment (start 59.125001 105.125001) (end 58.125001 105.125001) (width 0.25) (layer B.Cu) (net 17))
 (segment (start 59.125001 105.125001) (end 61.374999 105.125001) (width 0.25) (layer B.Cu) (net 17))
 (segment (start 57.5 97.96) (end 55 95.46) (width 0.25) (layer B.Cu) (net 17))
 (segment (start 57.738589 105.125001) (end 58.5 105.125001) (width 0.25) (layer B.Cu) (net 17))
 (segment (start 53 109.86359) (end 57.738589 105.125001) (width 0.25) (layer B.Cu) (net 17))
 (segment (start 53 116) (end 53 109.86359) (width 0.25) (layer B.Cu) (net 17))
 (segment (start 55.5 118.5) (end 53 116) (width 0.25) (layer B.Cu) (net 17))
 (segment (start 53.04 95.46) (end 55 95.46) (width 0.25) (layer B.Cu) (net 17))
 (segment (start 51.5 97) (end 53.04 95.46) (width 0.25) (layer B.Cu) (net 17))
 (segment (start 51.5 117.5) (end 51.5 97) (width 0.25) (layer B.Cu) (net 17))
 (segment (start 52.5 118.5) (end 51.5 117.5) (width 0.25) (layer B.Cu) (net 17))
 (segment (start 55.5 118.5) (end 52.5 118.5) (width 0.25) (layer B.Cu) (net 17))
 (segment (start 67.079999 124.874999) (end 70.410003 124.874999) (width 0.25) (layer B.Cu) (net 18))
 (segment (start 55.5 126.12) (end 57.804988 128.424988) (width 0.25) (layer B.Cu) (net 18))
 (segment (start 63.53001 128.424988) (end 67.079999 124.874999) (width 0.25) (layer B.Cu) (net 18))
 (segment (start 57.804988 128.424988) (end 63.53001 128.424988) (width 0.25) (layer B.Cu) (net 18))
 (segment (start 72.125001 123.160001) (end 72.125001 110.045001) (width 0.25) (layer B.Cu) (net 18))
 (segment (start 70.410003 124.874999) (end 72.125001 123.160001) (width 0.25) (layer B.Cu) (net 18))
 (segment (start 72.125001 110.045001) (end 70 107.92) (width 0.25) (layer B.Cu) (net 18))
 (segment (start 71 114) (end 70 113) (width 0.25) (layer F.Cu) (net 19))
 (segment (start 71 119) (end 71 114) (width 0.25) (layer F.Cu) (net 19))
 (segment (start 73.125001 82.085001) (end 70 78.96) (width 0.25) (layer B.Cu) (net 20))
 (segment (start 73.125001 96.494999) (end 73.125001 82.085001) (width 0.25) (layer B.Cu) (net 20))
 (segment (start 72 97.62) (end 73.125001 96.494999) (width 0.25) (layer B.Cu) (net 20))
 (segment (start 51.97499 82.59499) (end 53.5 84.12) (width 0.25) (layer F.Cu) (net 8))
 (segment (start 51.97499 71.52501) (end 51.97499 82.59499) (width 0.25) (layer F.Cu) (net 8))
 (segment (start 72.625001 70.540001) (end 70.665002 72.5) (width 0.25) (layer B.Cu) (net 8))
 (segment (start 70.665002 72.5) (end 66.5 72.5) (width 0.25) (layer B.Cu) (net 8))
 (segment (start 72.625001 69.459999) (end 72.625001 70.540001) (width 0.25) (layer B.Cu) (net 8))
 (segment (start 68.165002 65) (end 72.625001 69.459999) (width 0.25) (layer B.Cu) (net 8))
 (segment (start 66 65) (end 68.165002 65) (width 0.25) (layer B.Cu) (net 8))
 (segment (start 51.97499 71.52501) (end 53.5 70) (width 0.25) (layer F.Cu) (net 8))
 (segment (start 56 74.5) (end 53.5 72) (width 0.25) (layer B.Cu) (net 8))
 (segment (start 64.5 74.5) (end 56 74.5) (width 0.25) (layer B.Cu) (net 8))
 (segment (start 53.5 72) (end 53.5 70) (width 0.25) (layer B.Cu) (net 8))
 (segment (start 66.5 72.5) (end 64.5 74.5) (width 0.25) (layer B.Cu) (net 8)))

